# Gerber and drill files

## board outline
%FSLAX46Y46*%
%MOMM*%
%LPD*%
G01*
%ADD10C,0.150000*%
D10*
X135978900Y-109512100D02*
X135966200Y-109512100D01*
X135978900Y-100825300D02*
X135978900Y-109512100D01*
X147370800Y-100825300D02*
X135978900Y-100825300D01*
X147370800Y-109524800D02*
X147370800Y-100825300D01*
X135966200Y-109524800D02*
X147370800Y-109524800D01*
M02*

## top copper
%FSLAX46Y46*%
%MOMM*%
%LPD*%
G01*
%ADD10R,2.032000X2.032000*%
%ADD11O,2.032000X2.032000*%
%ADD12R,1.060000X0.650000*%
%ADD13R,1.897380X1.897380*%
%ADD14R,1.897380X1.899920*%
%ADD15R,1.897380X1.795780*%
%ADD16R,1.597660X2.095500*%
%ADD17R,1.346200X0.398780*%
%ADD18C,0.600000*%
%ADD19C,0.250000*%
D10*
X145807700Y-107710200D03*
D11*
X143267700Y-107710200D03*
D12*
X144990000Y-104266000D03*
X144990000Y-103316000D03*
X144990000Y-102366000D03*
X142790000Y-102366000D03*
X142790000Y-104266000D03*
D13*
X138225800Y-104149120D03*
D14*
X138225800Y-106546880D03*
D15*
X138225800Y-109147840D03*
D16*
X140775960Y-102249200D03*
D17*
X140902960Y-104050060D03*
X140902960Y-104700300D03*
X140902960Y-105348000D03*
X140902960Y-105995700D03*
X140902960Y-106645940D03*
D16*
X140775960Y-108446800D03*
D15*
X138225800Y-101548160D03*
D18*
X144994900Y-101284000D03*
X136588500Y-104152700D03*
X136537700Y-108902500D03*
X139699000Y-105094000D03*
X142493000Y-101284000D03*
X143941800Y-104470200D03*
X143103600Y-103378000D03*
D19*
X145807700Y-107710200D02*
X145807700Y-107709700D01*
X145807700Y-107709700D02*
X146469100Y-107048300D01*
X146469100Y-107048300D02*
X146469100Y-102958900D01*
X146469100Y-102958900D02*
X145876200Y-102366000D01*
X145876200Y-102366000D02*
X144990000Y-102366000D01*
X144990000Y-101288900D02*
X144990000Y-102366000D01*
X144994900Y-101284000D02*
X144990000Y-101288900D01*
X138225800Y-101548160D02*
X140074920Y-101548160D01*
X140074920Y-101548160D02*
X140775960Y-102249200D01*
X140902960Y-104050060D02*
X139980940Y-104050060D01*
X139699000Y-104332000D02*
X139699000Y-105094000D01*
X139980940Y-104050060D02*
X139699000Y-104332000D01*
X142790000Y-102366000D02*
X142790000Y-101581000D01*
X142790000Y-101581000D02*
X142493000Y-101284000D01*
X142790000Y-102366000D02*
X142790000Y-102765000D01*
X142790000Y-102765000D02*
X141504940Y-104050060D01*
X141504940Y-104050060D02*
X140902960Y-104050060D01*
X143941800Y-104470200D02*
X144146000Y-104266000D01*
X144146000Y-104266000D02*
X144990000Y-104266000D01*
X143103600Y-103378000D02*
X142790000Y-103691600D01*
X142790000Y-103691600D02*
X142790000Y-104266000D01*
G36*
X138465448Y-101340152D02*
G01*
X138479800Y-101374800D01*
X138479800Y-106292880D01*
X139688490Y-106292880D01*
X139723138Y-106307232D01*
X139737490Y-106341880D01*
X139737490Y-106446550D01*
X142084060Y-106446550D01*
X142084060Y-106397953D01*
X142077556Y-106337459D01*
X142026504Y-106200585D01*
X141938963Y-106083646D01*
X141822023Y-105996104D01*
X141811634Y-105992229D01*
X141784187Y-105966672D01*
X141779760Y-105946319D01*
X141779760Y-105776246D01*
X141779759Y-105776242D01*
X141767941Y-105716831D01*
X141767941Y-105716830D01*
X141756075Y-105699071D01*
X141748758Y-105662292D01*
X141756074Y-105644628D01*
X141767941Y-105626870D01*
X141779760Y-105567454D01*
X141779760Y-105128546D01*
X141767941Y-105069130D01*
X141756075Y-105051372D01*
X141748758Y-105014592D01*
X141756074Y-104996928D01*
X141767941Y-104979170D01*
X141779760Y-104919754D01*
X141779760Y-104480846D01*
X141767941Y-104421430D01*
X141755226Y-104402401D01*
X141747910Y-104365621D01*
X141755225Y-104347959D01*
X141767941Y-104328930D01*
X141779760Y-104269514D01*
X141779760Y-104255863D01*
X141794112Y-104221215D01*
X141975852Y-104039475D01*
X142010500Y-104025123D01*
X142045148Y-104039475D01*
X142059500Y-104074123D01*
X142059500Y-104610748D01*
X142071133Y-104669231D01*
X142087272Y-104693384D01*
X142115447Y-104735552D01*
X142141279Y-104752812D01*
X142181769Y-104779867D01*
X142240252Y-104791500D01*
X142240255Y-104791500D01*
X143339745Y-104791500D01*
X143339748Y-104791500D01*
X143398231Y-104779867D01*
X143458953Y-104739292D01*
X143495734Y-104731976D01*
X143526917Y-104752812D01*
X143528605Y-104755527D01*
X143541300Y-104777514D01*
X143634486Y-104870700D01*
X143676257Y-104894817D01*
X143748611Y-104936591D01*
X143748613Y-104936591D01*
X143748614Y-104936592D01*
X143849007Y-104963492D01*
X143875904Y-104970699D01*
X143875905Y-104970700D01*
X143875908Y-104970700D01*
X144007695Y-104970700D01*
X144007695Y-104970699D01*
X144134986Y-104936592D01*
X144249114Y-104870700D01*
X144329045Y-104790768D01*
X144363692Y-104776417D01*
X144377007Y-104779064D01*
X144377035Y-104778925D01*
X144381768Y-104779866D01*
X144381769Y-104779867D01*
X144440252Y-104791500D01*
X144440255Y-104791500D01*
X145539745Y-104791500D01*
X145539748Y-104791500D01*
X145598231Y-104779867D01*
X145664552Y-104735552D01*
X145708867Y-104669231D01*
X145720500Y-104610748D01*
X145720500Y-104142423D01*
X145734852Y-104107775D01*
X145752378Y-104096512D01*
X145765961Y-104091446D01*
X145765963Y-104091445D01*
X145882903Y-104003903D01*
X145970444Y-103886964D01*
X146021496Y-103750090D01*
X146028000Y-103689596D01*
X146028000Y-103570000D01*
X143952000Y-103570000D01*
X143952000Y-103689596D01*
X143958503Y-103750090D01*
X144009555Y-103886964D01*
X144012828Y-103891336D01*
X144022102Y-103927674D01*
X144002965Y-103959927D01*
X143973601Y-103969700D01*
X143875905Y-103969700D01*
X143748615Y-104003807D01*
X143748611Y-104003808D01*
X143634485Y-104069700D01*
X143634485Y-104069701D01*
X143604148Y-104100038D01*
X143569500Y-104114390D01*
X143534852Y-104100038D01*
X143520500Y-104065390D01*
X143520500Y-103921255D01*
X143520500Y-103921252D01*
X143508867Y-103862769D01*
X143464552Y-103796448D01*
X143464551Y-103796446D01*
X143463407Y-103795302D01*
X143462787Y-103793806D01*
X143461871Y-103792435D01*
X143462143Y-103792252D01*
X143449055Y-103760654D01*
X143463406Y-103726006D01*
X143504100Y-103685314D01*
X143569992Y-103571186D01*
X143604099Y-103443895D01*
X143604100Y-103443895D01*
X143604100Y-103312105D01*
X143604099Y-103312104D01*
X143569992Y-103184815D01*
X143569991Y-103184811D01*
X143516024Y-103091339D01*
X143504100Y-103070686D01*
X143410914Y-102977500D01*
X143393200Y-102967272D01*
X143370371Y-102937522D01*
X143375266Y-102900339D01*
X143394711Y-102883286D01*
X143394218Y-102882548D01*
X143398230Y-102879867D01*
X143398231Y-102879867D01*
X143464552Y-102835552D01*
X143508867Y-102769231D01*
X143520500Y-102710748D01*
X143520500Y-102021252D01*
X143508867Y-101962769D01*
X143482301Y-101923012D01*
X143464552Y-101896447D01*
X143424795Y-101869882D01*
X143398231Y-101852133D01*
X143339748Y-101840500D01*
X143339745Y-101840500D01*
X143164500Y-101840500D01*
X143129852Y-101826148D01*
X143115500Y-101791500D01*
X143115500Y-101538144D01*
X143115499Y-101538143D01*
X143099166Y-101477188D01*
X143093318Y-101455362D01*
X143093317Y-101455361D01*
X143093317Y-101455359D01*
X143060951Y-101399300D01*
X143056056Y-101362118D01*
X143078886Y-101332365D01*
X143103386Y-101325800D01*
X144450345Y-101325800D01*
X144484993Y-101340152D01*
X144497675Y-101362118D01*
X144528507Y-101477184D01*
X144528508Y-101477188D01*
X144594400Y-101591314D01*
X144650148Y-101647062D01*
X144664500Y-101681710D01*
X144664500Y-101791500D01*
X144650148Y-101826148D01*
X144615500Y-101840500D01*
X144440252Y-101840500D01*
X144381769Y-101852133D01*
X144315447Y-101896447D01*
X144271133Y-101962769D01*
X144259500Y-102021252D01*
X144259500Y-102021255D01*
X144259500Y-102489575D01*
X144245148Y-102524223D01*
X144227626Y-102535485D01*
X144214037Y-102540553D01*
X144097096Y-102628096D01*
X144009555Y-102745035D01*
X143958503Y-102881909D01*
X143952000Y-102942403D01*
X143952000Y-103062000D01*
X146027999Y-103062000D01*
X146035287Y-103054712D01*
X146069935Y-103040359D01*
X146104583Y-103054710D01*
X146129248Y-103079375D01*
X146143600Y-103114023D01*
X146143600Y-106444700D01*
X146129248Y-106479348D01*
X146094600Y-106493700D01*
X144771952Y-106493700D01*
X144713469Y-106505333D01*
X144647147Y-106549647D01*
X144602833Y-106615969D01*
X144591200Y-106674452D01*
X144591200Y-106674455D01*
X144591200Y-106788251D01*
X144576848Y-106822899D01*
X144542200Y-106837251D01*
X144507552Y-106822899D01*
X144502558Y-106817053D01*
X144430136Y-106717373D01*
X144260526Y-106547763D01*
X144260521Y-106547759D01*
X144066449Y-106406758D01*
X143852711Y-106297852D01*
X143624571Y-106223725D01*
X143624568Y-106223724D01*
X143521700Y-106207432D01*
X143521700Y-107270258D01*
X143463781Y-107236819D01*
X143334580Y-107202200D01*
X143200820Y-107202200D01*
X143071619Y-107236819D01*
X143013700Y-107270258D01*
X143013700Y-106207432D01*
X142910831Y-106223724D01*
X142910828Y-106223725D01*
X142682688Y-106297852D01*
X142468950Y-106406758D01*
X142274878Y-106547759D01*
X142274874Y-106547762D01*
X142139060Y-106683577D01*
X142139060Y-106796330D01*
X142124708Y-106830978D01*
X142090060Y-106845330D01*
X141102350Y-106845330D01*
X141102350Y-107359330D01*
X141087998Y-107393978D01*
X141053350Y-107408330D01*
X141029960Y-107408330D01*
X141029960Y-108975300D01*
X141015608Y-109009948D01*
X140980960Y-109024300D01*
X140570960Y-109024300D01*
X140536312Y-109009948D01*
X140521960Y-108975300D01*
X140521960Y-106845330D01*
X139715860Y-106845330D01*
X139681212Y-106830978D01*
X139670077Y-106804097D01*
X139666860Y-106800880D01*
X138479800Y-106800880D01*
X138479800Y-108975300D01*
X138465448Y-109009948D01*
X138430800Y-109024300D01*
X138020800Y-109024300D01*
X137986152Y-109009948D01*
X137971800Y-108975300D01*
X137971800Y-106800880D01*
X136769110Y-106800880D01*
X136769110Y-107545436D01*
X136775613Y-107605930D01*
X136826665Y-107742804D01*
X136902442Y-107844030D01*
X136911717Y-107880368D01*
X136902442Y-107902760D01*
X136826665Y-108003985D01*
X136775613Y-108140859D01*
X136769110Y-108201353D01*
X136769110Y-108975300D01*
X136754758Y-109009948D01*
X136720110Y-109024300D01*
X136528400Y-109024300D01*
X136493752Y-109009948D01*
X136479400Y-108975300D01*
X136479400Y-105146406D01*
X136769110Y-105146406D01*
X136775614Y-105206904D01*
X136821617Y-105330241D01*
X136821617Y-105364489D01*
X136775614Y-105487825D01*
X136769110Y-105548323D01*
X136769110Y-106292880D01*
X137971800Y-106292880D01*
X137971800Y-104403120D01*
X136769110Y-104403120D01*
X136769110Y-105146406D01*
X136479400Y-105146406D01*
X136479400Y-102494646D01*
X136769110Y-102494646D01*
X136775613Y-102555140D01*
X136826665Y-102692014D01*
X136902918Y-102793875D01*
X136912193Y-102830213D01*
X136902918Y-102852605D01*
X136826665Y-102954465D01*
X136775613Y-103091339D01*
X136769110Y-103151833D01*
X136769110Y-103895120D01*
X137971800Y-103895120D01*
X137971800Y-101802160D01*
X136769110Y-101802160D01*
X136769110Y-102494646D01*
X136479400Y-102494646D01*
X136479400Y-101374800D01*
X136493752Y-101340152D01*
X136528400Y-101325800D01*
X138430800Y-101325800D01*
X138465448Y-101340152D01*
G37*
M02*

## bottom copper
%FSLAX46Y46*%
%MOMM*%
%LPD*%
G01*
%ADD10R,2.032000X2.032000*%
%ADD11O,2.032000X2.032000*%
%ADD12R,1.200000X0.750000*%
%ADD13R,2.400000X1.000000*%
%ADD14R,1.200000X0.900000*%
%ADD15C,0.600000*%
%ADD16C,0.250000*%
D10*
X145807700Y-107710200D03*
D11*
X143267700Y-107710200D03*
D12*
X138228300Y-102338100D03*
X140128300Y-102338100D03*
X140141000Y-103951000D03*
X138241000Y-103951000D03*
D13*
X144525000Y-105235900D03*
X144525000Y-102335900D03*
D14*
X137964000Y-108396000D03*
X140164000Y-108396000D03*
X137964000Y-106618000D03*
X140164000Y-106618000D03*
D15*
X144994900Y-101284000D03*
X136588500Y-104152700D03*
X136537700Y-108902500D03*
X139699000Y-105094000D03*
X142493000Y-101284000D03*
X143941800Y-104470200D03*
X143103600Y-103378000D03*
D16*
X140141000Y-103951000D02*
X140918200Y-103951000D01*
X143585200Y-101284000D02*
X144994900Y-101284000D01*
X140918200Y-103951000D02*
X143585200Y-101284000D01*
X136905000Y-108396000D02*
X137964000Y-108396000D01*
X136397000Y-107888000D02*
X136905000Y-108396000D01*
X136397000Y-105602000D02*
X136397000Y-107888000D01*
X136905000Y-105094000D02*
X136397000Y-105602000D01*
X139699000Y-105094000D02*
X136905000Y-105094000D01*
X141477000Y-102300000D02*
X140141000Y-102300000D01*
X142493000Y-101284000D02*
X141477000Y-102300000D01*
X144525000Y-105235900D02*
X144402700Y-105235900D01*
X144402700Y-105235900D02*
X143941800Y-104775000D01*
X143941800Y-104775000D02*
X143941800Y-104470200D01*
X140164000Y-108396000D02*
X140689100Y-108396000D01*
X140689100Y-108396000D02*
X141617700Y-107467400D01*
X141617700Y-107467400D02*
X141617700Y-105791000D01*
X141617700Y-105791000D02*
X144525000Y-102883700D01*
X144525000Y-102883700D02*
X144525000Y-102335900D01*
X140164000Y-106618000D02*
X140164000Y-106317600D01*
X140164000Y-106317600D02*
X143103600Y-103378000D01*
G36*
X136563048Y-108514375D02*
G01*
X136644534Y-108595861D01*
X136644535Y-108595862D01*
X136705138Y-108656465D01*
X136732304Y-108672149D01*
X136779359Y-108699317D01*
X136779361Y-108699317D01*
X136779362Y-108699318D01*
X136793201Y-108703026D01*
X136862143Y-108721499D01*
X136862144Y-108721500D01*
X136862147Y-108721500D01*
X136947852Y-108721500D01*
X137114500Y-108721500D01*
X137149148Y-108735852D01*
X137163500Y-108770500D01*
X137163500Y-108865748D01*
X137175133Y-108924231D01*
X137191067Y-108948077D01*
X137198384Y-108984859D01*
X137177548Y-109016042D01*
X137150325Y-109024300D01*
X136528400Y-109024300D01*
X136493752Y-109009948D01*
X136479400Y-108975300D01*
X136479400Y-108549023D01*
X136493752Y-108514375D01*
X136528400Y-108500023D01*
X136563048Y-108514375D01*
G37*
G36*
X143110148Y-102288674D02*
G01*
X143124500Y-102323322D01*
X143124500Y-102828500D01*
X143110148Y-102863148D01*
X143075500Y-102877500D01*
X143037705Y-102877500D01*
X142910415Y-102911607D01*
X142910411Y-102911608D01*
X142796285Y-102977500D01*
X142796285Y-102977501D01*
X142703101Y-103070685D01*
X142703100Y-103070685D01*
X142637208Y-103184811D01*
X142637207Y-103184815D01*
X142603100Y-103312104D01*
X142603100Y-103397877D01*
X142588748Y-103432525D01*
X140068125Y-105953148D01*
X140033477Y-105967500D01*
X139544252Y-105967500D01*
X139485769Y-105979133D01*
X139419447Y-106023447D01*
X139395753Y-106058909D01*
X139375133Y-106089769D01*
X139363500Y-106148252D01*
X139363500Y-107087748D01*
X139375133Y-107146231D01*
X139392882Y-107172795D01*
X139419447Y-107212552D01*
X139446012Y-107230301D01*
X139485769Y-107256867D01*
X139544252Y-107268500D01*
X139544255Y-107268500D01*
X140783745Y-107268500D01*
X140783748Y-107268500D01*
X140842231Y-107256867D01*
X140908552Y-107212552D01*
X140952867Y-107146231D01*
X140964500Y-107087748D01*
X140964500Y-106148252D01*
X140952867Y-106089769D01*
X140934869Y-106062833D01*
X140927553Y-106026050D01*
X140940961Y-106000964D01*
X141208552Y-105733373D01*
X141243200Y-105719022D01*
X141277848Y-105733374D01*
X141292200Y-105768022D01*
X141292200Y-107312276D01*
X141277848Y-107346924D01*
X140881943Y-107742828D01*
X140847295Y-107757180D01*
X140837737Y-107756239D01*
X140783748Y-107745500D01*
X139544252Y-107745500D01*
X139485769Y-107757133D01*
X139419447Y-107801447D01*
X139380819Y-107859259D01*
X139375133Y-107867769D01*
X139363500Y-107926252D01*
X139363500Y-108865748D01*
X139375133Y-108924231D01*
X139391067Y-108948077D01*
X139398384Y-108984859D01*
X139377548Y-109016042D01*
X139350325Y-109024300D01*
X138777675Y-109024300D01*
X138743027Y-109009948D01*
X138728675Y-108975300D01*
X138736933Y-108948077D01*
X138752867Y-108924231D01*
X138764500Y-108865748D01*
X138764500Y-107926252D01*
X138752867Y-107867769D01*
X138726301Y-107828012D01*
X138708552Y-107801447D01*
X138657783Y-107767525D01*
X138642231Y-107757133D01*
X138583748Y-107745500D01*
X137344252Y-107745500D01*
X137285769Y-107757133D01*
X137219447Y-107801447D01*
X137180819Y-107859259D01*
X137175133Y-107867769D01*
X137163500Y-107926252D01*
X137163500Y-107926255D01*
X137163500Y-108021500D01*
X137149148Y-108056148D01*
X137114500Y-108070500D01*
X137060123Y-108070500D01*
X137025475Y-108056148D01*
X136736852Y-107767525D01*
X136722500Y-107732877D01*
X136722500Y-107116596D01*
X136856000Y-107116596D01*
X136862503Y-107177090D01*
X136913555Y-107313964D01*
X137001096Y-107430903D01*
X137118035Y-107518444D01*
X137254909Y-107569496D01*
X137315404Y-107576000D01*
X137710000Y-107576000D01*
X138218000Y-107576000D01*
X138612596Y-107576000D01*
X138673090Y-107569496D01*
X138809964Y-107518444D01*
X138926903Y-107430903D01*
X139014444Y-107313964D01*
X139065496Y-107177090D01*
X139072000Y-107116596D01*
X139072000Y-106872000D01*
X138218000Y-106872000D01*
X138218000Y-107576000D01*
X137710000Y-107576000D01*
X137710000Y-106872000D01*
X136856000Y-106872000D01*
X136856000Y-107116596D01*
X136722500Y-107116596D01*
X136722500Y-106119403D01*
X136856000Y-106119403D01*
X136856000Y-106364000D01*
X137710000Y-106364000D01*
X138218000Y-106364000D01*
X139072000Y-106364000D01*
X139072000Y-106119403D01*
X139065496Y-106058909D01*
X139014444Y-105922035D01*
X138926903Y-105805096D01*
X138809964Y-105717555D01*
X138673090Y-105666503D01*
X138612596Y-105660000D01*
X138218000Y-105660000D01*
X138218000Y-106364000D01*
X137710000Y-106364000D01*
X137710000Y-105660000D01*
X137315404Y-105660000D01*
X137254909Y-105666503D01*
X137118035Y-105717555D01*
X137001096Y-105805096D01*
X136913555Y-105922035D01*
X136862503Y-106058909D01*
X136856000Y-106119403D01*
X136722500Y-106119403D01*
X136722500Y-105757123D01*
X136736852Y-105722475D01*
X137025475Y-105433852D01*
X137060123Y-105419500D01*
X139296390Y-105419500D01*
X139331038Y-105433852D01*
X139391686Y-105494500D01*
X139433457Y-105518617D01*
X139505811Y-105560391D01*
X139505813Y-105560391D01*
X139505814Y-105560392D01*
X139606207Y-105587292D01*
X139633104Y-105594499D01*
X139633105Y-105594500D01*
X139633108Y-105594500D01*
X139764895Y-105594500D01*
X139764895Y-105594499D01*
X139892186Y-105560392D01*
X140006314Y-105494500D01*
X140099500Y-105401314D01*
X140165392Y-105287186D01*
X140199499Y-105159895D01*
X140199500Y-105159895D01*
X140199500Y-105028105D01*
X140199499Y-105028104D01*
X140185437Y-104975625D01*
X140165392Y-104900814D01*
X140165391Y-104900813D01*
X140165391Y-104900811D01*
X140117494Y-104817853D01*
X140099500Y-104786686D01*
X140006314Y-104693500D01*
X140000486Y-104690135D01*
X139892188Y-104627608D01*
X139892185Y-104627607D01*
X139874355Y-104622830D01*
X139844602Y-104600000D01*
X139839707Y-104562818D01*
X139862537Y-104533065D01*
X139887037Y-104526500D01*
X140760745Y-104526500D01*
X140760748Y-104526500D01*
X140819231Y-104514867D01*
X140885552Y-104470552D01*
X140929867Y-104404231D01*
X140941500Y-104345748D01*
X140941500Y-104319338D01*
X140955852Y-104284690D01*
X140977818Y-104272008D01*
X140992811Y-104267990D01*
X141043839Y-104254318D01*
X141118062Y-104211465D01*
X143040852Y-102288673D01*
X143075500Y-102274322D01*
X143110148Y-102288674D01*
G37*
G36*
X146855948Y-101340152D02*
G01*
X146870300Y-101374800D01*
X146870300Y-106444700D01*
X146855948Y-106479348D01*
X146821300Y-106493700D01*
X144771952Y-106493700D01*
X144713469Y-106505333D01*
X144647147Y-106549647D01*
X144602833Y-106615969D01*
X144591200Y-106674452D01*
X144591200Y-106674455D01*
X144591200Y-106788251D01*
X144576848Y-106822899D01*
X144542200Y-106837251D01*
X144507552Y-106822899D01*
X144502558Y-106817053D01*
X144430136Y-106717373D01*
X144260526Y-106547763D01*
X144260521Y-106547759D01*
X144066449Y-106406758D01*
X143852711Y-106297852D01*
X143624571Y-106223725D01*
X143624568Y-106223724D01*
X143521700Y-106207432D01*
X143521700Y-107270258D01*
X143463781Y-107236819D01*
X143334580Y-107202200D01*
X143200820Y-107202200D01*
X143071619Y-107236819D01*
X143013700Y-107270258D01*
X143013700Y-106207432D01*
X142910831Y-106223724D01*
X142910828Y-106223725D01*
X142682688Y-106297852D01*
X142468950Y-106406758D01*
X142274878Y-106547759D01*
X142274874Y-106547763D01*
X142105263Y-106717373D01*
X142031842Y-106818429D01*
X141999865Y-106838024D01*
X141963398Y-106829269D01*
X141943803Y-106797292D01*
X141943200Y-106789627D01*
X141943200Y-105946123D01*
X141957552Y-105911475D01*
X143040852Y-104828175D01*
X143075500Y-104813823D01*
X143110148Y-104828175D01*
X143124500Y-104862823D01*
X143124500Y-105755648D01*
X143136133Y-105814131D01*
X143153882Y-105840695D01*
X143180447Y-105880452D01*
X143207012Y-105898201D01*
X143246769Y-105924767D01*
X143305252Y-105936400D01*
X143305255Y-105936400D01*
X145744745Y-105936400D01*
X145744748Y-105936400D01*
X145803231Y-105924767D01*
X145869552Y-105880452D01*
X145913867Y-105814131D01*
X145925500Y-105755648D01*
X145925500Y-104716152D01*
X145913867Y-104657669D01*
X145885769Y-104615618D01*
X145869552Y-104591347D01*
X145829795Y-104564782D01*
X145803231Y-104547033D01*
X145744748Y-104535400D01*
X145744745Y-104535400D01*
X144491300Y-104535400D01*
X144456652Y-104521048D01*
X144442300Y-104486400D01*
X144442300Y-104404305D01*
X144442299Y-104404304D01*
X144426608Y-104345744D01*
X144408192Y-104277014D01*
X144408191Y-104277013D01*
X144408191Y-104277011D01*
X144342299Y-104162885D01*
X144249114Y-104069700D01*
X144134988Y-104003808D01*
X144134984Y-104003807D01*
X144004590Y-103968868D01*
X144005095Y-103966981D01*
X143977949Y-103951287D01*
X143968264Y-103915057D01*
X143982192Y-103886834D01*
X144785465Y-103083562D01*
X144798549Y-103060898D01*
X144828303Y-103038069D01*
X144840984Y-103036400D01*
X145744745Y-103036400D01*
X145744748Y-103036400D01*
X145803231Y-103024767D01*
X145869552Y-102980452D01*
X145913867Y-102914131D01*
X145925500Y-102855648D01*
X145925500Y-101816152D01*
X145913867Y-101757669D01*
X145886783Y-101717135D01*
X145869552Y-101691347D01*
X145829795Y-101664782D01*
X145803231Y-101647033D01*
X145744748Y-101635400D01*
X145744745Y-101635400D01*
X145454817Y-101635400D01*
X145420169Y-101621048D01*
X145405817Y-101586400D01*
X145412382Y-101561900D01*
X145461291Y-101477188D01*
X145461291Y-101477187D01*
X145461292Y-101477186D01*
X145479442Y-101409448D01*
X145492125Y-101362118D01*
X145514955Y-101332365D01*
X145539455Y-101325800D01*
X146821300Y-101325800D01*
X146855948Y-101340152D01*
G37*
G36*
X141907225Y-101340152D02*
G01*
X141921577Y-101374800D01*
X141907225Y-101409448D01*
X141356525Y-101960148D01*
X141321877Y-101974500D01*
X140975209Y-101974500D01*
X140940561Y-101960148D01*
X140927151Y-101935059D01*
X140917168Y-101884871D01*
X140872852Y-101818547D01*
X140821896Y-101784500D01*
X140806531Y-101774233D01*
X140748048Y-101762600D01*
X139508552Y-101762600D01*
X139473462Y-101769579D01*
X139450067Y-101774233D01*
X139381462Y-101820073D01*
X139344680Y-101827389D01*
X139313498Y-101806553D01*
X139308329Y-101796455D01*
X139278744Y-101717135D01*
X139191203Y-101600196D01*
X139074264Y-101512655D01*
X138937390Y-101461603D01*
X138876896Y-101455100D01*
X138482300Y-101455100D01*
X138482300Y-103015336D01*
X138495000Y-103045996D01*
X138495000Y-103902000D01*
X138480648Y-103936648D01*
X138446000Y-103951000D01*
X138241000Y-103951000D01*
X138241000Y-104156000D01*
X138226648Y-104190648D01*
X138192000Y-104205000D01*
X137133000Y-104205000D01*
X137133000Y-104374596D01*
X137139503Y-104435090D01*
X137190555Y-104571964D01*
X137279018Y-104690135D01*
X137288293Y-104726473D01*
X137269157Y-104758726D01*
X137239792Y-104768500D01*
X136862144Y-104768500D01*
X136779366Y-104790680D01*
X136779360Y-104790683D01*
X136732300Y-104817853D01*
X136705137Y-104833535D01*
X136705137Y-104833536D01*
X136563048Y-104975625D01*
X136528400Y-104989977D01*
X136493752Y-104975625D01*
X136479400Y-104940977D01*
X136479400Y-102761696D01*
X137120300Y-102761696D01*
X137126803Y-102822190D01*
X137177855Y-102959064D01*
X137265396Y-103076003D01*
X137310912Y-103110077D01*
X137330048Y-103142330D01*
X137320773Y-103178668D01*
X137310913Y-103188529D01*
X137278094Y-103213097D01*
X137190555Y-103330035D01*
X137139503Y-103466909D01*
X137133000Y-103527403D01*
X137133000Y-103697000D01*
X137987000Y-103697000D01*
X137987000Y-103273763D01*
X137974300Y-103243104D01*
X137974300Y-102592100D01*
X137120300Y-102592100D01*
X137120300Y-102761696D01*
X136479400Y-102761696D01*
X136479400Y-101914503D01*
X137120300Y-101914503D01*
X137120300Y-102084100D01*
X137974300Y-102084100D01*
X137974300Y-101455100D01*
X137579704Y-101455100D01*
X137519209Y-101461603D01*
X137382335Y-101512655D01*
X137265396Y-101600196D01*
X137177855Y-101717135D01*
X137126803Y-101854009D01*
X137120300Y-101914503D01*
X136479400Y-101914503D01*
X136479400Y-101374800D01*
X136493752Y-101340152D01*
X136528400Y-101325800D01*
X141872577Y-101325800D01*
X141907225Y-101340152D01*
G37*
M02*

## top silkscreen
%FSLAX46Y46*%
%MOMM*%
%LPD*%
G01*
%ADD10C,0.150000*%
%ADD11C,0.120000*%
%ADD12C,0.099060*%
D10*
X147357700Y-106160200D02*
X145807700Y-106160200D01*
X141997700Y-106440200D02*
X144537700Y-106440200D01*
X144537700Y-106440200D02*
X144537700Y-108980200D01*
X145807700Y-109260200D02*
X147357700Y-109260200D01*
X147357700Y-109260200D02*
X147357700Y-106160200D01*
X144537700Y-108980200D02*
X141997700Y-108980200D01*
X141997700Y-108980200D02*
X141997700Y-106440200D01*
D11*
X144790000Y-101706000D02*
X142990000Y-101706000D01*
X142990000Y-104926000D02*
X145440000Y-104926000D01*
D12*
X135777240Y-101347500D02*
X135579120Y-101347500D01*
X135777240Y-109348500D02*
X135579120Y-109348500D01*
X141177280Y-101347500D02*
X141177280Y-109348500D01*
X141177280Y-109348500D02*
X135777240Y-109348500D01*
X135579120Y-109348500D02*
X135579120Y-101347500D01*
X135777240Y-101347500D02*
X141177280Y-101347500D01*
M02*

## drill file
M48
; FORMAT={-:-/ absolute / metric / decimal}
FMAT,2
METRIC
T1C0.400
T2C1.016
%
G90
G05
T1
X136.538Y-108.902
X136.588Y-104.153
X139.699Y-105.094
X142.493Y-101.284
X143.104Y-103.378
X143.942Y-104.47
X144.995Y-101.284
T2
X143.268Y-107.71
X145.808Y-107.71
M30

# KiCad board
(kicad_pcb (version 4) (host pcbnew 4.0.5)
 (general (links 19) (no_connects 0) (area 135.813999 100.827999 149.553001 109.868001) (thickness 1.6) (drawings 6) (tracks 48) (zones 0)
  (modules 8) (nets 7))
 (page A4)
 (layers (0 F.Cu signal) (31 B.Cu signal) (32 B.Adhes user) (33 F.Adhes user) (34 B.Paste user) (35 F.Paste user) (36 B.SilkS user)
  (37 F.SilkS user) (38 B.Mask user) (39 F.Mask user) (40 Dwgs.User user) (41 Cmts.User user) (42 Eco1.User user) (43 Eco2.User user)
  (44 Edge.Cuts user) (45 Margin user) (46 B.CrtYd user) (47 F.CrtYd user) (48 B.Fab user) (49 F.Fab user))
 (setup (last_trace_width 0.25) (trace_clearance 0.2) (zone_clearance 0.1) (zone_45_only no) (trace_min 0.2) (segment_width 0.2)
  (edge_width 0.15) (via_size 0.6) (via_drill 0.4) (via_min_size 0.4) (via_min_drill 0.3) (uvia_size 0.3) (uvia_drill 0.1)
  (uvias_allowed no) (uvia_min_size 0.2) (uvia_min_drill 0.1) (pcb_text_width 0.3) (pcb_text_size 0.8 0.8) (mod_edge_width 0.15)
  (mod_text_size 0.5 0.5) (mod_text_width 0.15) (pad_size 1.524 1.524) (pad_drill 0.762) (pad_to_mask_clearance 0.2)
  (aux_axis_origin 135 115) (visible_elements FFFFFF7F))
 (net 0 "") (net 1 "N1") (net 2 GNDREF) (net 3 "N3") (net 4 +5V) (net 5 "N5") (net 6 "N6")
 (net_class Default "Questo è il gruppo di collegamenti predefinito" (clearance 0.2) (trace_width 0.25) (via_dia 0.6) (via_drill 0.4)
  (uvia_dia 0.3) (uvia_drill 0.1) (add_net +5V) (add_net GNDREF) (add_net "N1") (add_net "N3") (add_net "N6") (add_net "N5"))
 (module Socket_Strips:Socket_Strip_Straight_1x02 (layer F.Cu) (at 145.8077 107.7102 180)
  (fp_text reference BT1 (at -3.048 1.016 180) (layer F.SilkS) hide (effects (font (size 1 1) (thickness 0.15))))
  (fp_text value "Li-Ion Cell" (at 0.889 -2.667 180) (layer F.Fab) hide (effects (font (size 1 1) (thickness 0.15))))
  (fp_line (start -1.55 1.55) (end 0 1.55) (layer F.SilkS) (width 0.15))
  (fp_line (start 3.81 1.27) (end 1.27 1.27) (layer F.SilkS) (width 0.15))
  (fp_line (start 1.27 1.27) (end 1.27 -1.27) (layer F.SilkS) (width 0.15))
  (fp_line (start 0 -1.55) (end -1.55 -1.55) (layer F.SilkS) (width 0.15))
  (fp_line (start -1.55 -1.55) (end -1.55 1.55) (layer F.SilkS) (width 0.15))
  (fp_line (start 1.27 -1.27) (end 3.81 -1.27) (layer F.SilkS) (width 0.15))
  (fp_line (start 3.81 -1.27) (end 3.81 1.27) (layer F.SilkS) (width 0.15))
  (pad 1 thru_hole rect (at 0 0 180) (size 2.032 2.032) (drill 1.016) (layers *.Cu *.Mask) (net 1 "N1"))
  (pad 2 thru_hole oval (at 2.54 0 180) (size 2.032 2.032) (drill 1.016) (layers *.Cu *.Mask) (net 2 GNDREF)))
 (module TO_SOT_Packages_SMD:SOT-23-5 (layer F.Cu) (at 143.89 103.316 180)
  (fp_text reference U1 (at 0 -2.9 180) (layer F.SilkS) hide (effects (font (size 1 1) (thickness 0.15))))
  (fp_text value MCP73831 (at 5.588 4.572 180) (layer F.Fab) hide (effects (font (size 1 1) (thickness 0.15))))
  (fp_line (start -0.9 1.61) (end 0.9 1.61) (layer F.SilkS) (width 0.12))
  (fp_line (start 0.9 -1.61) (end -1.55 -1.61) (layer F.SilkS) (width 0.12))
  (pad 1 smd rect (at -1.1 -0.95 180) (size 1.06 0.65) (layers F.Cu F.Paste F.Mask) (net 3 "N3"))
  (pad 2 smd rect (at -1.1 0 180) (size 1.06 0.65) (layers F.Cu F.Paste F.Mask) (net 2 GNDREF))
  (pad 3 smd rect (at -1.1 0.95 180) (size 1.06 0.65) (layers F.Cu F.Paste F.Mask) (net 1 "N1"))
  (pad 4 smd rect (at 1.1 0.95 180) (size 1.06 0.65) (layers F.Cu F.Paste F.Mask) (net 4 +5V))
  (pad 5 smd rect (at 1.1 -0.95 180) (size 1.06 0.65) (layers F.Cu F.Paste F.Mask) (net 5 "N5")))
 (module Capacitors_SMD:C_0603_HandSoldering (layer B.Cu) (at 139.1783 102.3381)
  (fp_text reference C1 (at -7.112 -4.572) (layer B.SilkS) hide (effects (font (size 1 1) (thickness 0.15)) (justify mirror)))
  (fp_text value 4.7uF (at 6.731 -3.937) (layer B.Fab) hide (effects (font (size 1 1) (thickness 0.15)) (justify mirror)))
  (pad 1 smd rect (at -0.95 0) (size 1.2 0.75) (layers B.Cu B.Paste B.Mask) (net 2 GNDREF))
  (pad 2 smd rect (at 0.95 0) (size 1.2 0.75) (layers B.Cu B.Paste B.Mask) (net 4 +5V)))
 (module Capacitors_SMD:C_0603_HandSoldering (layer B.Cu) (at 139.191 103.951 180)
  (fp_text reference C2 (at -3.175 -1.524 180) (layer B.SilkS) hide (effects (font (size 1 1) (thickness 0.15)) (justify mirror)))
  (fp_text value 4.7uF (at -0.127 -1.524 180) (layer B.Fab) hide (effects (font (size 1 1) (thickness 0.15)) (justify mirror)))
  (pad 1 smd rect (at -0.95 0 180) (size 1.2 0.75) (layers B.Cu B.Paste B.Mask) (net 1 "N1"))
  (pad 2 smd rect (at 0.95 0 180) (size 1.2 0.75) (layers B.Cu B.Paste B.Mask) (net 2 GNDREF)))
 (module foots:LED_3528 (layer B.Cu) (at 144.525 103.7859 180)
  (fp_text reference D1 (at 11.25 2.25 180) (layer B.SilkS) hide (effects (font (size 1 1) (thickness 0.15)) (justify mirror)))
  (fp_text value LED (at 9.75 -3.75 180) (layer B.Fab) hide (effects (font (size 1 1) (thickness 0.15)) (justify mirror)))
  (pad 1 smd rect (at 0 -1.45 180) (size 2.4 1) (layers B.Cu B.Paste B.Mask) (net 3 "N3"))
  (pad 2 smd rect (at 0 1.45 180) (size 2.4 1) (layers B.Cu B.Paste B.Mask) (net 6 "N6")))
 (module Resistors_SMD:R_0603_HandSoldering (layer B.Cu) (at 139.064 108.396)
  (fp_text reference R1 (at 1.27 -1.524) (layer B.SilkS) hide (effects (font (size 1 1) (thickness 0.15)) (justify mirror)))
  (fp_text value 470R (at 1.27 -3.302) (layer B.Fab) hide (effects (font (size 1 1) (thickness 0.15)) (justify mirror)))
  (pad 1 smd rect (at -1.1 0) (size 1.2 0.9) (layers B.Cu B.Paste B.Mask) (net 4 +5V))
  (pad 2 smd rect (at 1.1 0) (size 1.2 0.9) (layers B.Cu B.Paste B.Mask) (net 6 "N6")))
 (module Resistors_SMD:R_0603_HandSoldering (layer B.Cu) (at 139.064 106.618)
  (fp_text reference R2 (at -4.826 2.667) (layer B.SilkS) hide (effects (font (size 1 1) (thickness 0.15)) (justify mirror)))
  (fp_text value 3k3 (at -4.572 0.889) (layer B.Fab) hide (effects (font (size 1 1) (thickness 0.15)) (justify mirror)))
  (pad 1 smd rect (at -1.1 0) (size 1.2 0.9) (layers B.Cu B.Paste B.Mask) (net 2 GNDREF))
  (pad 2 smd rect (at 1.1 0) (size 1.2 0.9) (layers B.Cu B.Paste B.Mask) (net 5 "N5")))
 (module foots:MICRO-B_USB (layer F.Cu) (at 136.778 105.348 270)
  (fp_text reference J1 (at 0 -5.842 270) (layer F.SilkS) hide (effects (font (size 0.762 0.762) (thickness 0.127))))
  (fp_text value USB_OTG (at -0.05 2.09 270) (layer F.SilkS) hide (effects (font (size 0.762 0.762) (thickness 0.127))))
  (fp_line (start -4.0005 1.00076) (end -4.0005 1.19888) (layer F.SilkS) (width 0.09906))
  (fp_line (start 4.0005 1.00076) (end 4.0005 1.19888) (layer F.SilkS) (width 0.09906))
  (fp_line (start -4.0005 -4.39928) (end 4.0005 -4.39928) (layer F.SilkS) (width 0.09906))
  (fp_line (start 4.0005 -4.39928) (end 4.0005 1.00076) (layer F.SilkS) (width 0.09906))
  (fp_line (start 4.0005 1.19888) (end -4.0005 1.19888) (layer F.SilkS) (width 0.09906))
  (fp_line (start -4.0005 1.00076) (end -4.0005 -4.39928) (layer F.SilkS) (width 0.09906))
  (pad 6 smd rect (at -1.19888 -1.4478 270) (size 1.89738 1.89738) (layers F.Cu F.Paste F.Mask) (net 2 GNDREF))
  (pad 6 smd rect (at 1.19888 -1.4478 270) (size 1.89992 1.89738) (layers F.Cu F.Paste F.Mask) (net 2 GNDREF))
  (pad 6 smd rect (at 3.79984 -1.4478 270) (size 1.79578 1.89738) (layers F.Cu F.Paste F.Mask) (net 2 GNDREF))
  (pad 6 smd rect (at -3.0988 -3.99796 270) (size 2.0955 1.59766) (layers F.Cu F.Paste F.Mask) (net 2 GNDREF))
  (pad 1 smd rect (at -1.29794 -4.12496 270) (size 0.39878 1.3462) (layers F.Cu F.Paste F.Mask) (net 4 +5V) (clearance 0.2032))
  (pad 2 smd rect (at -0.6477 -4.12496 270) (size 0.39878 1.3462) (layers F.Cu F.Paste F.Mask) (clearance 0.2032))
  (pad 3 smd rect (at 0 -4.12496 270) (size 0.39878 1.3462) (layers F.Cu F.Paste F.Mask) (clearance 0.2032))
  (pad 4 smd rect (at 0.6477 -4.12496 270) (size 0.39878 1.3462) (layers F.Cu F.Paste F.Mask) (clearance 0.2032))
  (pad 5 smd rect (at 1.29794 -4.12496 270) (size 0.39878 1.3462) (layers F.Cu F.Paste F.Mask) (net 2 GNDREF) (clearance 0.2032))
  (pad 6 smd rect (at 3.0988 -3.99796 270) (size 2.0955 1.59766) (layers F.Cu F.Paste F.Mask) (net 2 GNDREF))
  (pad 6 smd rect (at -3.79984 -1.4478 270) (size 1.79578 1.89738) (layers F.Cu F.Paste F.Mask) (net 2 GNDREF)))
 (gr_line (start 135.9789 109.5121) (end 135.9662 109.5121) (angle 90) (layer Edge.Cuts) (width 0.15))
 (gr_line (start 135.9789 100.8253) (end 135.9789 109.5121) (angle 90) (layer Edge.Cuts) (width 0.15))
 (gr_line (start 147.3708 100.8253) (end 135.9789 100.8253) (angle 90) (layer Edge.Cuts) (width 0.15))
 (gr_line (start 147.3708 109.5248) (end 147.3708 100.8253) (angle 90) (layer Edge.Cuts) (width 0.15))
 (gr_line (start 135.9662 109.5248) (end 147.3708 109.5248) (angle 90) (layer Edge.Cuts) (width 0.15))
 (segment (start 145.8077 107.7102) (end 145.8077 107.7097) (width 0.25) (layer F.Cu) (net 1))
 (segment (start 145.8077 107.7097) (end 146.4691 107.0483) (width 0.25) (layer F.Cu) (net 1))
 (segment (start 146.4691 107.0483) (end 146.4691 102.9589) (width 0.25) (layer F.Cu) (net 1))
 (segment (start 146.4691 102.9589) (end 145.8762 102.366) (width 0.25) (layer F.Cu) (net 1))
 (segment (start 145.8762 102.366) (end 144.99 102.366) (width 0.25) (layer F.Cu) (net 1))
 (segment (start 140.141 103.951) (end 140.9182 103.951) (width 0.25) (layer B.Cu) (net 1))
 (segment (start 144.99 101.2889) (end 144.99 102.366) (width 0.25) (layer F.Cu) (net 1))
 (segment (start 144.9949 101.284) (end 144.99 101.2889) (width 0.25) (layer F.Cu) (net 1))
 (via (at 144.9949 101.284) (size 0.6) (drill 0.4) (layers F.Cu B.Cu) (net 1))
 (segment (start 143.5852 101.284) (end 144.9949 101.284) (width 0.25) (layer B.Cu) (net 1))
 (segment (start 140.9182 103.951) (end 143.5852 101.284) (width 0.25) (layer B.Cu) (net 1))
 (via (at 136.5885 104.1527) (size 0.6) (drill 0.4) (layers F.Cu B.Cu) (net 2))
 (via (at 136.5377 108.9025) (size 0.6) (drill 0.4) (layers F.Cu B.Cu) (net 2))
 (segment (start 138.2258 101.54816) (end 140.07492 101.54816) (width 0.25) (layer F.Cu) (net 2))
 (segment (start 140.07492 101.54816) (end 140.77596 102.2492) (width 0.25) (layer F.Cu) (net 2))
 (segment (start 140.90296 104.05006) (end 139.98094 104.05006) (width 0.25) (layer F.Cu) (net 4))
 (segment (start 136.905 108.396) (end 137.964 108.396) (width 0.25) (layer B.Cu) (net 4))
 (segment (start 136.397 107.888) (end 136.905 108.396) (width 0.25) (layer B.Cu) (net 4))
 (segment (start 136.397 105.602) (end 136.397 107.888) (width 0.25) (layer B.Cu) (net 4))
 (segment (start 136.905 105.094) (end 136.397 105.602) (width 0.25) (layer B.Cu) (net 4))
 (segment (start 139.699 105.094) (end 136.905 105.094) (width 0.25) (layer B.Cu) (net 4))
 (via (at 139.699 105.094) (size 0.6) (drill 0.4) (layers F.Cu B.Cu) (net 4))
 (segment (start 139.699 104.332) (end 139.699 105.094) (width 0.25) (layer F.Cu) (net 4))
 (segment (start 139.98094 104.05006) (end 139.699 104.332) (width 0.25) (layer F.Cu) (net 4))
 (segment (start 142.79 102.366) (end 142.79 101.581) (width 0.25) (layer F.Cu) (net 4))
 (segment (start 141.477 102.3) (end 140.141 102.3) (width 0.25) (layer B.Cu) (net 4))
 (segment (start 142.493 101.284) (end 141.477 102.3) (width 0.25) (layer B.Cu) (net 4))
 (via (at 142.493 101.284) (size 0.6) (drill 0.4) (layers F.Cu B.Cu) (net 4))
 (segment (start 142.79 101.581) (end 142.493 101.284) (width 0.25) (layer F.Cu) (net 4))
 (segment (start 142.79 102.366) (end 142.79 102.765) (width 0.25) (layer F.Cu) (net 4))
 (segment (start 142.79 102.765) (end 141.50494 104.05006) (width 0.25) (layer F.Cu) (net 4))
 (segment (start 141.50494 104.05006) (end 140.90296 104.05006) (width 0.25) (layer F.Cu) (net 4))
 (segment (start 144.525 105.2359) (end 144.4027 105.2359) (width 0.25) (layer B.Cu) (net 3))
 (segment (start 144.4027 105.2359) (end 143.9418 104.775) (width 0.25) (layer B.Cu) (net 3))
 (segment (start 143.9418 104.775) (end 143.9418 104.4702) (width 0.25) (layer B.Cu) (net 3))
 (via (at 143.9418 104.4702) (size 0.6) (drill 0.4) (layers F.Cu B.Cu) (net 3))
 (segment (start 143.9418 104.4702) (end 144.146 104.266) (width 0.25) (layer F.Cu) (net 3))
 (segment (start 144.146 104.266) (end 144.99 104.266) (width 0.25) (layer F.Cu) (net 3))
 (segment (start 140.164 108.396) (end 140.6891 108.396) (width 0.25) (layer B.Cu) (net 6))
 (segment (start 140.6891 108.396) (end 141.6177 107.4674) (width 0.25) (layer B.Cu) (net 6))
 (segment (start 141.6177 107.4674) (end 141.6177 105.791) (width 0.25) (layer B.Cu) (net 6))
 (segment (start 141.6177 105.791) (end 144.525 102.8837) (width 0.25) (layer B.Cu) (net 6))
 (segment (start 144.525 102.8837) (end 144.525 102.3359) (width 0.25) (layer B.Cu) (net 6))
 (segment (start 140.164 106.618) (end 140.164 106.3176) (width 0.25) (layer B.Cu) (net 5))
 (segment (start 140.164 106.3176) (end 143.1036 103.378) (width 0.25) (layer B.Cu) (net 5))
 (via (at 143.1036 103.378) (size 0.6) (drill 0.4) (layers F.Cu B.Cu) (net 5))
 (segment (start 143.1036 103.378) (end 142.79 103.6916) (width 0.25) (layer F.Cu) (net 5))
 (segment (start 142.79 103.6916) (end 142.79 104.266) (width 0.25) (layer F.Cu) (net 5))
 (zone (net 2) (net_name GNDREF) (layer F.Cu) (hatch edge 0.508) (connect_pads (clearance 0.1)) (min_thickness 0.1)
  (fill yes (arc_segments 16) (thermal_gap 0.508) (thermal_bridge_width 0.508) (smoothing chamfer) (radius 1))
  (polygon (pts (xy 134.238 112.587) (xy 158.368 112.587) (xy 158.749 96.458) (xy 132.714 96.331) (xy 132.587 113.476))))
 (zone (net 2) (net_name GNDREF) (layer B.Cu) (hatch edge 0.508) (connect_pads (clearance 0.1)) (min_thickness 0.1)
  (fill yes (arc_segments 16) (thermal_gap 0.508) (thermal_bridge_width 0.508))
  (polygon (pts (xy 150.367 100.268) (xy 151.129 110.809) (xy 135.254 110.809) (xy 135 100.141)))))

